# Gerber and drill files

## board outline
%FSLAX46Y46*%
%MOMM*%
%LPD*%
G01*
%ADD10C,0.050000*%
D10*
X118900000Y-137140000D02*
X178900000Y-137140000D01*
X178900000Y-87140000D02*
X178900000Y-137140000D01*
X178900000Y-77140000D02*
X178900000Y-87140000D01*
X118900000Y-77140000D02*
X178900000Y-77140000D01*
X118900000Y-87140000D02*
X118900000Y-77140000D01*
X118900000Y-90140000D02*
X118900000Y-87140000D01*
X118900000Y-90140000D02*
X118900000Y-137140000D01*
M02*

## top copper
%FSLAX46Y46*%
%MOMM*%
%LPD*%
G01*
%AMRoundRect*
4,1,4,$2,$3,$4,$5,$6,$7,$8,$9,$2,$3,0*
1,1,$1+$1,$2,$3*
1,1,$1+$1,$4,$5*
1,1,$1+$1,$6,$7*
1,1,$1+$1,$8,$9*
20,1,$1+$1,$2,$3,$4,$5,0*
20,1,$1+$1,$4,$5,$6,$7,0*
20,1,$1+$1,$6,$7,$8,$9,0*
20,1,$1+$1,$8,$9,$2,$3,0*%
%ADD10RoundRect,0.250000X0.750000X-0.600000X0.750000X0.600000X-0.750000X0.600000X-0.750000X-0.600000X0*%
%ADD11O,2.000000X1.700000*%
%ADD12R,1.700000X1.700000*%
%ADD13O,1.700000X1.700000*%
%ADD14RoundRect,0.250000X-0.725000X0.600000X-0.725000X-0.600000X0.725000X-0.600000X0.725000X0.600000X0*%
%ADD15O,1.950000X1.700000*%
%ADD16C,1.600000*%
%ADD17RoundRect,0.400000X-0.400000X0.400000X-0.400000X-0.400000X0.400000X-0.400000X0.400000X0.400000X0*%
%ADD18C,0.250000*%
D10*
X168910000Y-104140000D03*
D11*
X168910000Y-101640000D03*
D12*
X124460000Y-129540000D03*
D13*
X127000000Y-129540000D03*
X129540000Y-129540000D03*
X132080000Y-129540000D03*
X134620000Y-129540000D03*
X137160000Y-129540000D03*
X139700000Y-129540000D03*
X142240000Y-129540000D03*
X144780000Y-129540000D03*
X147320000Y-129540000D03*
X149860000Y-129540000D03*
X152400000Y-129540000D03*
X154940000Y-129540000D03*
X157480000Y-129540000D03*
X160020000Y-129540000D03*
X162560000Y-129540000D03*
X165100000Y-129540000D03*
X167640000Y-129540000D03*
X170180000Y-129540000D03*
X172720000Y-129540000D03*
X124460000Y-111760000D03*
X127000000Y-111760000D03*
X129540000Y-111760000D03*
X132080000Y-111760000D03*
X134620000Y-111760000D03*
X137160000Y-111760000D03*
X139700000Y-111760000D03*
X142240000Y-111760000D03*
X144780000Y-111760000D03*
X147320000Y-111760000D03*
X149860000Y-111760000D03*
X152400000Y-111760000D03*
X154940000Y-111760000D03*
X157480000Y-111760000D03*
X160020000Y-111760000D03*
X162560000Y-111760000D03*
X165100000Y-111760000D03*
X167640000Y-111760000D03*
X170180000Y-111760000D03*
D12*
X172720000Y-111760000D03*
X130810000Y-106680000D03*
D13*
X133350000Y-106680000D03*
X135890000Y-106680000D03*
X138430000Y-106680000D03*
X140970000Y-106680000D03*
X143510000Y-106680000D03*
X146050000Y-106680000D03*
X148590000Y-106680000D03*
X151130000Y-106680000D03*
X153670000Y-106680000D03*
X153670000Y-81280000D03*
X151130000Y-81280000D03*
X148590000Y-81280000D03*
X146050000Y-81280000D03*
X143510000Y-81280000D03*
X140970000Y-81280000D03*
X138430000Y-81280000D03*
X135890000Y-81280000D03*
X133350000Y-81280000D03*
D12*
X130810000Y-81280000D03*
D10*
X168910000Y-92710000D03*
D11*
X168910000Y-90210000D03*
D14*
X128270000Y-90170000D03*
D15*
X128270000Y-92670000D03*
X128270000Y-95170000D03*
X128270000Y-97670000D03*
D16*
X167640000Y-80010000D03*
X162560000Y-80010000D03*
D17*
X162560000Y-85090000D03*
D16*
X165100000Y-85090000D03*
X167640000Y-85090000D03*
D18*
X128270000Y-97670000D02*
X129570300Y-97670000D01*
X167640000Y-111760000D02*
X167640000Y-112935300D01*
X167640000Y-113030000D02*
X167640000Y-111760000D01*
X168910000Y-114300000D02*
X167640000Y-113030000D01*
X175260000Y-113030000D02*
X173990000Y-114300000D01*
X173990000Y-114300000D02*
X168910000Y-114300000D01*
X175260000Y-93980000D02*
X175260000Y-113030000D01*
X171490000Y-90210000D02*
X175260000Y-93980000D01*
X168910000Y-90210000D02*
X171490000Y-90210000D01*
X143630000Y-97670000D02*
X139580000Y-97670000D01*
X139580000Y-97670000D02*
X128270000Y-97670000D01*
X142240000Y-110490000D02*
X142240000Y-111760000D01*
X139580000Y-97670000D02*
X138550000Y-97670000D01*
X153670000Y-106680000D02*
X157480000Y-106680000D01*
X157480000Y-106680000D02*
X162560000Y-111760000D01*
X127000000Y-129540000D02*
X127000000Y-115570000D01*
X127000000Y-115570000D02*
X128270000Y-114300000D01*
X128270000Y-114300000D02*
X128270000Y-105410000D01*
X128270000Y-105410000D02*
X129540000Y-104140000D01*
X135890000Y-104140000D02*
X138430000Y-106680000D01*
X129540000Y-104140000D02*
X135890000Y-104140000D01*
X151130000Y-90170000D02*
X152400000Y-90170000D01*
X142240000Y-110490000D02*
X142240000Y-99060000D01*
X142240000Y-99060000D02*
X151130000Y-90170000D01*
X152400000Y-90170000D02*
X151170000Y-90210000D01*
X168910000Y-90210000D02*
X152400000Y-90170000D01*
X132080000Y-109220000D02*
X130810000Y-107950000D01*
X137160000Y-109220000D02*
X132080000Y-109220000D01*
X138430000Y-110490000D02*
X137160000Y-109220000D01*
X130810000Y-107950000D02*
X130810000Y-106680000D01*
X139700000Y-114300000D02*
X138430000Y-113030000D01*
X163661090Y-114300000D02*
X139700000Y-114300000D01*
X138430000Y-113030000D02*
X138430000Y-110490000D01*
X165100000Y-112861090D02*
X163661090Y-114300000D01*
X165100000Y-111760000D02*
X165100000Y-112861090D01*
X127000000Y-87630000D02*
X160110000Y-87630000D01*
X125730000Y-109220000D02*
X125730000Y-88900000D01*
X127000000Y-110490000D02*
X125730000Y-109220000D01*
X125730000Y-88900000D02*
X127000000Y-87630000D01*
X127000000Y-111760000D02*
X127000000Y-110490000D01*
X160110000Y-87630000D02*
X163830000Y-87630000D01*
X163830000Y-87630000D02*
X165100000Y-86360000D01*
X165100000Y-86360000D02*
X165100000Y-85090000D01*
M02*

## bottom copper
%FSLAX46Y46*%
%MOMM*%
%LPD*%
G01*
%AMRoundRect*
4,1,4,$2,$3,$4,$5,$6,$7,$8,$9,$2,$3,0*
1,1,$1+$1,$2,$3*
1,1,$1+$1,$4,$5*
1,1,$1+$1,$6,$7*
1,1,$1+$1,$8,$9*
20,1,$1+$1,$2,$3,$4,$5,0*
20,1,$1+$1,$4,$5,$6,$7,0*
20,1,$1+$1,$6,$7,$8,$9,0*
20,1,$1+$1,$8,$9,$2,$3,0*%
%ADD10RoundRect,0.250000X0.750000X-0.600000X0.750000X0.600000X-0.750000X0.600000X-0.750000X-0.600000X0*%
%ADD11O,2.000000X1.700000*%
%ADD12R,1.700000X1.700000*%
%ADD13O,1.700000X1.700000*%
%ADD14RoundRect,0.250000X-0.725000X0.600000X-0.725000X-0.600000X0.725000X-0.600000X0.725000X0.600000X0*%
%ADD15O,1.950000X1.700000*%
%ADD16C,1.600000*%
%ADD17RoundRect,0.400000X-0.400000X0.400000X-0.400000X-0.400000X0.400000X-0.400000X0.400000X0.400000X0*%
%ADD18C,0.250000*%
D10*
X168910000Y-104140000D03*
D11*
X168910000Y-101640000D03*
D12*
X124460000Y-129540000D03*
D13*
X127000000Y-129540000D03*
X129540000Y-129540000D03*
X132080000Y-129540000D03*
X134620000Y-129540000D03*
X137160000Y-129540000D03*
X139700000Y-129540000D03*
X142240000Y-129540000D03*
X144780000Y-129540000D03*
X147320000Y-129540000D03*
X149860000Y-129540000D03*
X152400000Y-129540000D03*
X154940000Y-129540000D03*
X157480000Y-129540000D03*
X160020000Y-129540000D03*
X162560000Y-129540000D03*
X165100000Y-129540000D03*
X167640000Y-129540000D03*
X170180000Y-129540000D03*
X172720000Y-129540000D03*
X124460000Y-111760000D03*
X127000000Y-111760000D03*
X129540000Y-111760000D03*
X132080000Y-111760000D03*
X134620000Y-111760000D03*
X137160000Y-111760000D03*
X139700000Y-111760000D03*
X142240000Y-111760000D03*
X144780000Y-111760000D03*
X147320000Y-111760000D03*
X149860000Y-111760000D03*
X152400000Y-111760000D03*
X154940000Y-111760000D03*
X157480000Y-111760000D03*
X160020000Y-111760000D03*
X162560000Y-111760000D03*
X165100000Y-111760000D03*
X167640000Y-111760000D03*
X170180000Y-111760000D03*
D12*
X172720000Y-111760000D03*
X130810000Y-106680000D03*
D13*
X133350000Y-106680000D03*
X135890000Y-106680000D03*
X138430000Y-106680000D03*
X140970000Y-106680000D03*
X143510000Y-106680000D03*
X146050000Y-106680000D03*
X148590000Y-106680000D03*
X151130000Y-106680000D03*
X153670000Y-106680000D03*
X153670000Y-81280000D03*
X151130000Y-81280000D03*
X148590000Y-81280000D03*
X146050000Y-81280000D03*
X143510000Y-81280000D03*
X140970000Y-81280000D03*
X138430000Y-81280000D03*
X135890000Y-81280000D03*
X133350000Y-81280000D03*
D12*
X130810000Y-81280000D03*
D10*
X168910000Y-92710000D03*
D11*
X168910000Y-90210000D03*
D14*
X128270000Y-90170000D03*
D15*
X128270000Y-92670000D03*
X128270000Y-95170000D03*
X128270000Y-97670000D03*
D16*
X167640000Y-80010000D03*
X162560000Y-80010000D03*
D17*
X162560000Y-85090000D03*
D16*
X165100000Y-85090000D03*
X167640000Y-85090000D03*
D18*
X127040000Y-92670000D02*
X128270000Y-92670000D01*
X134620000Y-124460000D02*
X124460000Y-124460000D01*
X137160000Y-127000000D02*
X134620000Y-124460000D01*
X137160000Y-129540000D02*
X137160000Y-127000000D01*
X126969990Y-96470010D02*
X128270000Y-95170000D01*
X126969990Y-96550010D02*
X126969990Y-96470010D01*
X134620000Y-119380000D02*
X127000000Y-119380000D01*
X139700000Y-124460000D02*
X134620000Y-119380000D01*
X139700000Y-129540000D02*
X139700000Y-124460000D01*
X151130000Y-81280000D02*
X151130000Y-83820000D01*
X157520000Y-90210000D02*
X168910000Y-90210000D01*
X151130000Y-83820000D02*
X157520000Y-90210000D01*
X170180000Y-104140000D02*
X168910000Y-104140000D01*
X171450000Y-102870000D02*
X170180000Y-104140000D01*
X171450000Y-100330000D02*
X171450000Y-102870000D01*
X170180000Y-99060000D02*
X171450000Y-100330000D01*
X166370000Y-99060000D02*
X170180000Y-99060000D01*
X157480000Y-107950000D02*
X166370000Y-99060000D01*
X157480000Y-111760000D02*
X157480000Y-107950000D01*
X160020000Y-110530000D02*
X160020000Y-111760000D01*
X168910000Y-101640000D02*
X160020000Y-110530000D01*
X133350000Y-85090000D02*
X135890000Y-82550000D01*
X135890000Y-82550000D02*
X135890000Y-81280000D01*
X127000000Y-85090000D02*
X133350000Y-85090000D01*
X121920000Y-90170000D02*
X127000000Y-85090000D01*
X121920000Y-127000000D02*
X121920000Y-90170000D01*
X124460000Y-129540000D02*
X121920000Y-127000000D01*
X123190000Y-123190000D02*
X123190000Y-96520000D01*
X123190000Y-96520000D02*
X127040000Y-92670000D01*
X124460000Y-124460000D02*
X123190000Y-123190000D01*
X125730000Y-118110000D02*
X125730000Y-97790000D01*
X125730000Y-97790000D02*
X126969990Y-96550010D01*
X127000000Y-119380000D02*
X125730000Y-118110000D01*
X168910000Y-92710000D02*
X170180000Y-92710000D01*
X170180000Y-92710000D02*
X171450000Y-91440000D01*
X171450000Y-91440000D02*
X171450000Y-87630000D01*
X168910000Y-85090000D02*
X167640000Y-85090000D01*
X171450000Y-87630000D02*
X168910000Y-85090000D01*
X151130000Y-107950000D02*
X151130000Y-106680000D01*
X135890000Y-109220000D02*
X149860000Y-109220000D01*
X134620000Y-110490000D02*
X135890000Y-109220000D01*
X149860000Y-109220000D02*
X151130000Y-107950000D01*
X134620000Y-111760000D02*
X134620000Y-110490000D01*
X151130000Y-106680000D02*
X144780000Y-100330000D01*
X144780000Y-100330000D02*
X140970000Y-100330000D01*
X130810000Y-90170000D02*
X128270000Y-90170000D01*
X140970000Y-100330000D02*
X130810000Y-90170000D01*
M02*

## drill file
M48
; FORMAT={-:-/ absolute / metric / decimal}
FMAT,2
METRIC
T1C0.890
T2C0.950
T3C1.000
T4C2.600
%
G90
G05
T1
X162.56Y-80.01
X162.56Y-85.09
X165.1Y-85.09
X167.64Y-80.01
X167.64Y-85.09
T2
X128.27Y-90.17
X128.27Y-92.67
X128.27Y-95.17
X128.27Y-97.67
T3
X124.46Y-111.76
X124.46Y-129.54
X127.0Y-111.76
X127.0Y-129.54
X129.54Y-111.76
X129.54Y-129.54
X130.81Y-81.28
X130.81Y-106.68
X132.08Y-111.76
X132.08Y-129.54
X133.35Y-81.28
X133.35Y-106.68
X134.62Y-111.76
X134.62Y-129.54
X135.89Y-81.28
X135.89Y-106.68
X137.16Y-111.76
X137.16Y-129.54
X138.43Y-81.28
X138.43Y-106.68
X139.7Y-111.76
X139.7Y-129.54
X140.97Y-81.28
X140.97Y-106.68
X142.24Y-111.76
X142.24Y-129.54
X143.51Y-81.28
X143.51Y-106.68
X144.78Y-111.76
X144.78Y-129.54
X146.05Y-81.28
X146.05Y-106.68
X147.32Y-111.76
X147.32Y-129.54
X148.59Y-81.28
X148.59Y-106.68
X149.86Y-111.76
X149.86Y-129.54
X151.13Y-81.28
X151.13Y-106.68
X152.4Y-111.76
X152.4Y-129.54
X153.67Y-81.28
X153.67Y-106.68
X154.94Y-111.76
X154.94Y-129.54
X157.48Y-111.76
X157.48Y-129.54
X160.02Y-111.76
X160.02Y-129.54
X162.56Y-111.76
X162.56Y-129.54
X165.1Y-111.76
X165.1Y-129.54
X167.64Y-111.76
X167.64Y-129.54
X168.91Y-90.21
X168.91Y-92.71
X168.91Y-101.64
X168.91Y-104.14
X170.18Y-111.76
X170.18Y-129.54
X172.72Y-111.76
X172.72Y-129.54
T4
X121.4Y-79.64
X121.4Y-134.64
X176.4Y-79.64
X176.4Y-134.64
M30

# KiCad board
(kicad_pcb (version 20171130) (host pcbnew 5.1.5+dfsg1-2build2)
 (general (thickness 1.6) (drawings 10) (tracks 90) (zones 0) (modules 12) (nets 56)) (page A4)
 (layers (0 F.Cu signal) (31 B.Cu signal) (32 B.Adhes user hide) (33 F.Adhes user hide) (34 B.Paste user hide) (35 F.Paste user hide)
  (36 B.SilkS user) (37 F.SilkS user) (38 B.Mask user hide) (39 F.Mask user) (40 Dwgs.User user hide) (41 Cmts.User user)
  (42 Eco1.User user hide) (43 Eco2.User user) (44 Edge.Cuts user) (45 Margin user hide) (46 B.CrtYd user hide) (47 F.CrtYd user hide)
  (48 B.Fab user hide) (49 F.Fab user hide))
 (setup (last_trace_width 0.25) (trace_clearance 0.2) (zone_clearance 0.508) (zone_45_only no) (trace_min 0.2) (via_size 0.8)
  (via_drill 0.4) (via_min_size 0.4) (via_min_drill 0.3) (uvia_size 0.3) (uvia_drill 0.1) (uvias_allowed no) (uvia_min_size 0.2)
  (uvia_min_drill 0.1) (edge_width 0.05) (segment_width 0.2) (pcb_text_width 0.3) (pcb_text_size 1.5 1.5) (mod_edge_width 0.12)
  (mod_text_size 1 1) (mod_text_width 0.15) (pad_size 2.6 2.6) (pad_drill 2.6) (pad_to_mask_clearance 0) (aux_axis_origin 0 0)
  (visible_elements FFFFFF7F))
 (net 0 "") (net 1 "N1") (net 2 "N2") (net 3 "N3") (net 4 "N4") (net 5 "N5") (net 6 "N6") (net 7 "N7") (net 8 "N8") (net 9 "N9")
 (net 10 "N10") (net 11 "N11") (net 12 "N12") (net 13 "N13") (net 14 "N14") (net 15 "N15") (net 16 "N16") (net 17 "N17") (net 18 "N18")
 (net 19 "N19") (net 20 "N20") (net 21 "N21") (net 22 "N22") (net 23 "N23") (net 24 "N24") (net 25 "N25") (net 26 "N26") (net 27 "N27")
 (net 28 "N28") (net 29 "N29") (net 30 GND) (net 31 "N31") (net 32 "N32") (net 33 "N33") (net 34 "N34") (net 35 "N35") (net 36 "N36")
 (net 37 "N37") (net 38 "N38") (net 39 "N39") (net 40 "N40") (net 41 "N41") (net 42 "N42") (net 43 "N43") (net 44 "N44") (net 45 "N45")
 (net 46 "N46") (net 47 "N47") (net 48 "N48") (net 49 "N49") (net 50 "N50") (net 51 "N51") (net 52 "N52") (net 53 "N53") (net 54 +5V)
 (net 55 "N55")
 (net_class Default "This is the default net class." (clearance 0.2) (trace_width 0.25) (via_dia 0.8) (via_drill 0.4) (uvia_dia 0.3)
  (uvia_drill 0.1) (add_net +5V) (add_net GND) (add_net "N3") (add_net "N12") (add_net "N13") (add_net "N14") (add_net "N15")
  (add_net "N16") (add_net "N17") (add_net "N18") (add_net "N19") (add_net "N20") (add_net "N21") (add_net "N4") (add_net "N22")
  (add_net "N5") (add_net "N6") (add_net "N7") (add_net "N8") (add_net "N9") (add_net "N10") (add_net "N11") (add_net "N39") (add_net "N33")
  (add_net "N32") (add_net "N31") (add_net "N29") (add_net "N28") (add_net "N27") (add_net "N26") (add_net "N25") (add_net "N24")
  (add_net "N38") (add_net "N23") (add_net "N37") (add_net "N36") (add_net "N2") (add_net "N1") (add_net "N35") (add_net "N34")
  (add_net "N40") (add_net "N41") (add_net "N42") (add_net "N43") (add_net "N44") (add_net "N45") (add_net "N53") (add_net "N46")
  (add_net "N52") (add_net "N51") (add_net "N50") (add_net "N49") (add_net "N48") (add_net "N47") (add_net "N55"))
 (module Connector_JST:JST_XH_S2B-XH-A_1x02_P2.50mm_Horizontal (layer F.Cu) (at 168.91 104.14 90)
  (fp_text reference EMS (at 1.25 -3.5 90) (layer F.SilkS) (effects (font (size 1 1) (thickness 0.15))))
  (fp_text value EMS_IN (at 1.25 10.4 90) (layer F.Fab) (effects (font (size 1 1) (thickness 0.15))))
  (pad 1 thru_hole roundrect (at 0 0 90) (size 1.7 2) (drill 1) (layers *.Cu *.Mask) (roundrect_rratio 0.147059) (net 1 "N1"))
  (pad 2 thru_hole oval (at 2.5 0 90) (size 1.7 2) (drill 1) (layers *.Cu *.Mask) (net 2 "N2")))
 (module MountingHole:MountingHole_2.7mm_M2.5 (layer F.Cu) (at 176.4 134.64)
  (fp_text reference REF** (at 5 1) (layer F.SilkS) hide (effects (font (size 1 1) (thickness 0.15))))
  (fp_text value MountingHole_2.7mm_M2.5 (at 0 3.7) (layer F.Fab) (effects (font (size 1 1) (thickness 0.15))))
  (pad "" np_thru_hole circle (at 0 0) (size 2.6 2.6) (drill 2.6) (layers *.Cu *.Mask)))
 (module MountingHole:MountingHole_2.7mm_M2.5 (layer F.Cu) (at 176.4 79.64)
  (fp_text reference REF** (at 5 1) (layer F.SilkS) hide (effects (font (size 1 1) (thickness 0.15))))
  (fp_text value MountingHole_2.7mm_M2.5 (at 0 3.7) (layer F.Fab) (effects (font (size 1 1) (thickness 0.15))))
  (pad "" np_thru_hole circle (at 0 0) (size 2.6 2.6) (drill 2.6) (layers *.Cu *.Mask)))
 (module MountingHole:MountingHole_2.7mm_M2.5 (layer F.Cu) (at 121.4 79.64)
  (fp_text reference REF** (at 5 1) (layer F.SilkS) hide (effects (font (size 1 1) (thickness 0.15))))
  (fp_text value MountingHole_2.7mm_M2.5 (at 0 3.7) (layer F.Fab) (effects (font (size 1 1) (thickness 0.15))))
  (pad "" np_thru_hole circle (at 0 0) (size 2.6 2.6) (drill 2.6) (layers *.Cu *.Mask)))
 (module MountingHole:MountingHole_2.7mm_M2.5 (layer B.Cu) (at 121.4 134.64)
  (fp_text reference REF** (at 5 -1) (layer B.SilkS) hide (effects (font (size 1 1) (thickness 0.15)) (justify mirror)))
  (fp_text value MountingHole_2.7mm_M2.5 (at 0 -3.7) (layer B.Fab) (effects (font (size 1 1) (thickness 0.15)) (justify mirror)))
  (pad "" np_thru_hole circle (at 0 0) (size 2.6 2.6) (drill 2.6) (layers *.Cu *.Mask)))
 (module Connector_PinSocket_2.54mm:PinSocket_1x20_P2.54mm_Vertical (layer F.Cu) (at 124.46 129.54 90)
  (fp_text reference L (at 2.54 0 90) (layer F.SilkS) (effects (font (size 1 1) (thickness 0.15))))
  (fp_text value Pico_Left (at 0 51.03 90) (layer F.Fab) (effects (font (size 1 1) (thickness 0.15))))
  (pad 1 thru_hole rect (at 0 0 90) (size 1.7 1.7) (drill 1) (layers *.Cu *.Mask) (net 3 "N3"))
  (pad 2 thru_hole oval (at 0 2.54 90) (size 1.7 1.7) (drill 1) (layers *.Cu *.Mask) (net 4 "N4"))
  (pad 3 thru_hole oval (at 0 5.08 90) (size 1.7 1.7) (drill 1) (layers *.Cu *.Mask) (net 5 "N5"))
  (pad 4 thru_hole oval (at 0 7.62 90) (size 1.7 1.7) (drill 1) (layers *.Cu *.Mask) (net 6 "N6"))
  (pad 5 thru_hole oval (at 0 10.16 90) (size 1.7 1.7) (drill 1) (layers *.Cu *.Mask) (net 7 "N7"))
  (pad 6 thru_hole oval (at 0 12.7 90) (size 1.7 1.7) (drill 1) (layers *.Cu *.Mask) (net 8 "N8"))
  (pad 7 thru_hole oval (at 0 15.24 90) (size 1.7 1.7) (drill 1) (layers *.Cu *.Mask) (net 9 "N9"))
  (pad 8 thru_hole oval (at 0 17.78 90) (size 1.7 1.7) (drill 1) (layers *.Cu *.Mask) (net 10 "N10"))
  (pad 9 thru_hole oval (at 0 20.32 90) (size 1.7 1.7) (drill 1) (layers *.Cu *.Mask) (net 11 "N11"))
  (pad 10 thru_hole oval (at 0 22.86 90) (size 1.7 1.7) (drill 1) (layers *.Cu *.Mask) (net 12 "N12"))
  (pad 11 thru_hole oval (at 0 25.4 90) (size 1.7 1.7) (drill 1) (layers *.Cu *.Mask) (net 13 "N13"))
  (pad 12 thru_hole oval (at 0 27.94 90) (size 1.7 1.7) (drill 1) (layers *.Cu *.Mask) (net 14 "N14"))
  (pad 13 thru_hole oval (at 0 30.48 90) (size 1.7 1.7) (drill 1) (layers *.Cu *.Mask) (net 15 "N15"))
  (pad 14 thru_hole oval (at 0 33.02 90) (size 1.7 1.7) (drill 1) (layers *.Cu *.Mask) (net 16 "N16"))
  (pad 15 thru_hole oval (at 0 35.56 90) (size 1.7 1.7) (drill 1) (layers *.Cu *.Mask) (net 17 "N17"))
  (pad 16 thru_hole oval (at 0 38.1 90) (size 1.7 1.7) (drill 1) (layers *.Cu *.Mask) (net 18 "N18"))
  (pad 17 thru_hole oval (at 0 40.64 90) (size 1.7 1.7) (drill 1) (layers *.Cu *.Mask) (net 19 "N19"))
  (pad 18 thru_hole oval (at 0 43.18 90) (size 1.7 1.7) (drill 1) (layers *.Cu *.Mask) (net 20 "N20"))
  (pad 19 thru_hole oval (at 0 45.72 90) (size 1.7 1.7) (drill 1) (layers *.Cu *.Mask) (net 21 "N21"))
  (pad 20 thru_hole oval (at 0 48.26 90) (size 1.7 1.7) (drill 1) (layers *.Cu *.Mask) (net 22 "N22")))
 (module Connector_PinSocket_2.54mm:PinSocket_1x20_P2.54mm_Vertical (layer F.Cu) (at 172.72 111.76 270)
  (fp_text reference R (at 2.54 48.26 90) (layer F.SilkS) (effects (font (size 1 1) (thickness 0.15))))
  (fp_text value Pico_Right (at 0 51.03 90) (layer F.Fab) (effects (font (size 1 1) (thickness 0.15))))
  (pad 20 thru_hole oval (at 0 48.26 270) (size 1.7 1.7) (drill 1) (layers *.Cu *.Mask) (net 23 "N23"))
  (pad 19 thru_hole oval (at 0 45.72 270) (size 1.7 1.7) (drill 1) (layers *.Cu *.Mask) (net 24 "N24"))
  (pad 18 thru_hole oval (at 0 43.18 270) (size 1.7 1.7) (drill 1) (layers *.Cu *.Mask) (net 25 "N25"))
  (pad 17 thru_hole oval (at 0 40.64 270) (size 1.7 1.7) (drill 1) (layers *.Cu *.Mask) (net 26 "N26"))
  (pad 16 thru_hole oval (at 0 38.1 270) (size 1.7 1.7) (drill 1) (layers *.Cu *.Mask) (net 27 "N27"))
  (pad 15 thru_hole oval (at 0 35.56 270) (size 1.7 1.7) (drill 1) (layers *.Cu *.Mask) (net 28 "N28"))
  (pad 14 thru_hole oval (at 0 33.02 270) (size 1.7 1.7) (drill 1) (layers *.Cu *.Mask) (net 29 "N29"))
  (pad 13 thru_hole oval (at 0 30.48 270) (size 1.7 1.7) (drill 1) (layers *.Cu *.Mask) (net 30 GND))
  (pad 12 thru_hole oval (at 0 27.94 270) (size 1.7 1.7) (drill 1) (layers *.Cu *.Mask) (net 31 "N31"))
  (pad 11 thru_hole oval (at 0 25.4 270) (size 1.7 1.7) (drill 1) (layers *.Cu *.Mask) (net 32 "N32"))
  (pad 10 thru_hole oval (at 0 22.86 270) (size 1.7 1.7) (drill 1) (layers *.Cu *.Mask) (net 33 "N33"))
  (pad 9 thru_hole oval (at 0 20.32 270) (size 1.7 1.7) (drill 1) (layers *.Cu *.Mask) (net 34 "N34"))
  (pad 8 thru_hole oval (at 0 17.78 270) (size 1.7 1.7) (drill 1) (layers *.Cu *.Mask) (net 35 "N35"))
  (pad 7 thru_hole oval (at 0 15.24 270) (size 1.7 1.7) (drill 1) (layers *.Cu *.Mask) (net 1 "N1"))
  (pad 6 thru_hole oval (at 0 12.7 270) (size 1.7 1.7) (drill 1) (layers *.Cu *.Mask) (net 2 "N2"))
  (pad 5 thru_hole oval (at 0 10.16 270) (size 1.7 1.7) (drill 1) (layers *.Cu *.Mask) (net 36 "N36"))
  (pad 4 thru_hole oval (at 0 7.62 270) (size 1.7 1.7) (drill 1) (layers *.Cu *.Mask) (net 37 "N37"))
  (pad 3 thru_hole oval (at 0 5.08 270) (size 1.7 1.7) (drill 1) (layers *.Cu *.Mask) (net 30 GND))
  (pad 2 thru_hole oval (at 0 2.54 270) (size 1.7 1.7) (drill 1) (layers *.Cu *.Mask) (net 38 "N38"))
  (pad 1 thru_hole rect (at 0 0 270) (size 1.7 1.7) (drill 1) (layers *.Cu *.Mask) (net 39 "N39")))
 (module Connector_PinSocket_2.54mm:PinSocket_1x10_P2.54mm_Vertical (layer F.Cu) (at 130.81 106.68 90)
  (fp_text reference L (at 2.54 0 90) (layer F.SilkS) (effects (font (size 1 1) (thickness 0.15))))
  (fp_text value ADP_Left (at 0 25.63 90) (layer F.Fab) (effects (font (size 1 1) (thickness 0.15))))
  (pad 1 thru_hole rect (at 0 0 90) (size 1.7 1.7) (drill 1) (layers *.Cu *.Mask) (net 37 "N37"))
  (pad 2 thru_hole oval (at 0 2.54 90) (size 1.7 1.7) (drill 1) (layers *.Cu *.Mask) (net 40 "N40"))
  (pad 3 thru_hole oval (at 0 5.08 90) (size 1.7 1.7) (drill 1) (layers *.Cu *.Mask) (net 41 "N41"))
  (pad 4 thru_hole oval (at 0 7.62 90) (size 1.7 1.7) (drill 1) (layers *.Cu *.Mask) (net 4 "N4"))
  (pad 5 thru_hole oval (at 0 10.16 90) (size 1.7 1.7) (drill 1) (layers *.Cu *.Mask) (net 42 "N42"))
  (pad 6 thru_hole oval (at 0 12.7 90) (size 1.7 1.7) (drill 1) (layers *.Cu *.Mask) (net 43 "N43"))
  (pad 7 thru_hole oval (at 0 15.24 90) (size 1.7 1.7) (drill 1) (layers *.Cu *.Mask) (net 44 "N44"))
  (pad 8 thru_hole oval (at 0 17.78 90) (size 1.7 1.7) (drill 1) (layers *.Cu *.Mask) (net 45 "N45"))
  (pad 9 thru_hole oval (at 0 20.32 90) (size 1.7 1.7) (drill 1) (layers *.Cu *.Mask) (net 27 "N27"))
  (pad 10 thru_hole oval (at 0 22.86 90) (size 1.7 1.7) (drill 1) (layers *.Cu *.Mask) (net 36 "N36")))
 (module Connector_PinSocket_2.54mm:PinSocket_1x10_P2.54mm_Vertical (layer F.Cu) (at 130.81 81.28 90)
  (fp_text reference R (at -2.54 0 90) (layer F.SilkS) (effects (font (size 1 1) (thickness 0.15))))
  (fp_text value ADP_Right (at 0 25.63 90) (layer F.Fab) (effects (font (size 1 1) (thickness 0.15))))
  (pad 10 thru_hole oval (at 0 22.86 90) (size 1.7 1.7) (drill 1) (layers *.Cu *.Mask) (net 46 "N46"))
  (pad 9 thru_hole oval (at 0 20.32 90) (size 1.7 1.7) (drill 1) (layers *.Cu *.Mask) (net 30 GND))
  (pad 8 thru_hole oval (at 0 17.78 90) (size 1.7 1.7) (drill 1) (layers *.Cu *.Mask) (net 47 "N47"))
  (pad 7 thru_hole oval (at 0 15.24 90) (size 1.7 1.7) (drill 1) (layers *.Cu *.Mask) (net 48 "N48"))
  (pad 6 thru_hole oval (at 0 12.7 90) (size 1.7 1.7) (drill 1) (layers *.Cu *.Mask) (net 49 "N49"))
  (pad 5 thru_hole oval (at 0 10.16 90) (size 1.7 1.7) (drill 1) (layers *.Cu *.Mask) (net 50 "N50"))
  (pad 4 thru_hole oval (at 0 7.62 90) (size 1.7 1.7) (drill 1) (layers *.Cu *.Mask) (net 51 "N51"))
  (pad 3 thru_hole oval (at 0 5.08 90) (size 1.7 1.7) (drill 1) (layers *.Cu *.Mask) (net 3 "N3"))
  (pad 2 thru_hole oval (at 0 2.54 90) (size 1.7 1.7) (drill 1) (layers *.Cu *.Mask) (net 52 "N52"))
  (pad 1 thru_hole rect (at 0 0 90) (size 1.7 1.7) (drill 1) (layers *.Cu *.Mask) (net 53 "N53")))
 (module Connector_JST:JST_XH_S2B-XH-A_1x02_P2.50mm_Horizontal (layer F.Cu) (at 168.91 92.71 90)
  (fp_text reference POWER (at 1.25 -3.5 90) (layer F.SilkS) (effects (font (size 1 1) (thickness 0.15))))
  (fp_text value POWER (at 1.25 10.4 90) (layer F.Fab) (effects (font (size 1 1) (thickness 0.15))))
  (pad 1 thru_hole roundrect (at 0 0 90) (size 1.7 2) (drill 1) (layers *.Cu *.Mask) (roundrect_rratio 0.1470588235294118) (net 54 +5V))
  (pad 2 thru_hole oval (at 2.5 0 90) (size 1.7 2) (drill 1) (layers *.Cu *.Mask) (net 30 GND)))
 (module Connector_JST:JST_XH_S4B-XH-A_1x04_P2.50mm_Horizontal (layer F.Cu) (at 128.27 90.17 270)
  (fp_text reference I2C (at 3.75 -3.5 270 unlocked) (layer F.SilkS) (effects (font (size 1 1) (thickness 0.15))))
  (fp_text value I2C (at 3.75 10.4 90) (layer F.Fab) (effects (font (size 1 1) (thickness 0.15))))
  (pad 1 thru_hole roundrect (at 0 0 270) (size 1.7 1.95) (drill 0.95) (layers *.Cu *.Mask) (roundrect_rratio 0.147059) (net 27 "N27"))
  (pad 2 thru_hole oval (at 2.5 0 270) (size 1.7 1.95) (drill 0.95) (layers *.Cu *.Mask) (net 8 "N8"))
  (pad 3 thru_hole oval (at 5 0 270) (size 1.7 1.95) (drill 0.95) (layers *.Cu *.Mask) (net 9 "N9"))
  (pad 4 thru_hole oval (at 7.5 0 270) (size 1.7 1.95) (drill 0.95) (layers *.Cu *.Mask) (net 30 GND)))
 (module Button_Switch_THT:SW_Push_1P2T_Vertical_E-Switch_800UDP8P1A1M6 (layer F.Cu) (at 162.56 85.09 90)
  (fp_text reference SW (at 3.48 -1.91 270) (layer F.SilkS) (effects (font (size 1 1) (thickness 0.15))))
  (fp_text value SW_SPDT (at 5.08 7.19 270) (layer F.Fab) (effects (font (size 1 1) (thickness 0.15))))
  (pad "" thru_hole circle (at 5.08 5.08 270) (size 1.6 1.6) (drill 0.89) (layers *.Cu *.Mask))
  (pad "" thru_hole circle (at 5.08 0 270) (size 1.6 1.6) (drill 0.89) (layers *.Cu *.Mask))
  (pad 1 thru_hole roundrect (at 0 0 270) (size 1.6 1.6) (drill 0.89) (layers *.Cu *.Mask) (roundrect_rratio 0.25) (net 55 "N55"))
  (pad 2 thru_hole circle (at 0 2.54 270) (size 1.6 1.6) (drill 0.89) (layers *.Cu *.Mask) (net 24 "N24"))
  (pad 3 thru_hole circle (at 0 5.08 270) (size 1.6 1.6) (drill 0.89) (layers *.Cu *.Mask) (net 54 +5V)))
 (gr_line (start 118.9 137.14) (end 178.9 137.14) (layer Edge.Cuts) (width 0.05))
 (gr_line (start 178.9 87.14) (end 178.9 137.14) (layer Edge.Cuts) (width 0.05))
 (gr_line (start 178.9 77.14) (end 178.9 87.14) (layer Edge.Cuts) (width 0.05))
 (gr_line (start 118.9 77.14) (end 178.9 77.14) (layer Edge.Cuts) (width 0.05))
 (gr_line (start 118.9 87.14) (end 118.9 77.14) (layer Edge.Cuts) (width 0.05))
 (gr_line (start 118.9 90.14) (end 118.9 87.14) (layer Edge.Cuts) (width 0.05))
 (gr_line (start 118.9 90.14) (end 118.9 137.14) (layer Edge.Cuts) (width 0.05))
 (segment (start 127.04 92.67) (end 128.27 92.67) (width 0.25) (layer B.Cu) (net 8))
 (segment (start 134.62 124.46) (end 124.46 124.46) (width 0.25) (layer B.Cu) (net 8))
 (segment (start 137.16 127) (end 134.62 124.46) (width 0.25) (layer B.Cu) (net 8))
 (segment (start 137.16 129.54) (end 137.16 127) (width 0.25) (layer B.Cu) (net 8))
 (segment (start 126.96999 96.47001) (end 128.27 95.17) (width 0.25) (layer B.Cu) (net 9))
 (segment (start 126.96999 96.55001) (end 126.96999 96.47001) (width 0.25) (layer B.Cu) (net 9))
 (segment (start 134.62 119.38) (end 127 119.38) (width 0.25) (layer B.Cu) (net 9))
 (segment (start 139.7 124.46) (end 134.62 119.38) (width 0.25) (layer B.Cu) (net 9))
 (segment (start 139.7 129.54) (end 139.7 124.46) (width 0.25) (layer B.Cu) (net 9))
 (segment (start 128.27 97.67) (end 129.5703 97.67) (width 0.25) (layer F.Cu) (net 30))
 (segment (start 167.64 111.76) (end 167.64 112.9353) (width 0.25) (layer F.Cu) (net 30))
 (segment (start 151.13 81.28) (end 151.13 83.82) (width 0.25) (layer B.Cu) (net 30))
 (segment (start 157.52 90.21) (end 168.91 90.21) (width 0.25) (layer B.Cu) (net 30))
 (segment (start 151.13 83.82) (end 157.52 90.21) (width 0.25) (layer B.Cu) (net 30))
 (segment (start 167.64 113.03) (end 167.64 111.76) (width 0.25) (layer F.Cu) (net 30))
 (segment (start 168.91 114.3) (end 167.64 113.03) (width 0.25) (layer F.Cu) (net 30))
 (segment (start 175.26 113.03) (end 173.99 114.3) (width 0.25) (layer F.Cu) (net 30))
 (segment (start 173.99 114.3) (end 168.91 114.3) (width 0.25) (layer F.Cu) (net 30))
 (segment (start 175.26 93.98) (end 175.26 113.03) (width 0.25) (layer F.Cu) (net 30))
 (segment (start 171.49 90.21) (end 175.26 93.98) (width 0.25) (layer F.Cu) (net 30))
 (segment (start 168.91 90.21) (end 171.49 90.21) (width 0.25) (layer F.Cu) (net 30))
 (segment (start 143.63 97.67) (end 139.58 97.67) (width 0.25) (layer F.Cu) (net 30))
 (segment (start 139.58 97.67) (end 128.27 97.67) (width 0.25) (layer F.Cu) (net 30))
 (segment (start 142.24 110.49) (end 142.24 111.76) (width 0.25) (layer F.Cu) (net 30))
 (segment (start 139.58 97.67) (end 138.55 97.67) (width 0.25) (layer F.Cu) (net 30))
 (segment (start 170.18 104.14) (end 168.91 104.14) (width 0.25) (layer B.Cu) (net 1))
 (segment (start 171.45 102.87) (end 170.18 104.14) (width 0.25) (layer B.Cu) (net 1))
 (segment (start 171.45 100.33) (end 171.45 102.87) (width 0.25) (layer B.Cu) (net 1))
 (segment (start 170.18 99.06) (end 171.45 100.33) (width 0.25) (layer B.Cu) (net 1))
 (segment (start 166.37 99.06) (end 170.18 99.06) (width 0.25) (layer B.Cu) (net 1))
 (segment (start 157.48 107.95) (end 166.37 99.06) (width 0.25) (layer B.Cu) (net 1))
 (segment (start 157.48 111.76) (end 157.48 107.95) (width 0.25) (layer B.Cu) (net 1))
 (segment (start 160.02 110.53) (end 160.02 111.76) (width 0.25) (layer B.Cu) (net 2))
 (segment (start 168.91 101.64) (end 160.02 110.53) (width 0.25) (layer B.Cu) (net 2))
 (segment (start 153.67 106.68) (end 157.48 106.68) (width 0.25) (layer F.Cu) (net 36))
 (segment (start 157.48 106.68) (end 162.56 111.76) (width 0.25) (layer F.Cu) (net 36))
 (segment (start 133.35 85.09) (end 135.89 82.55) (width 0.25) (layer B.Cu) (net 3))
 (segment (start 135.89 82.55) (end 135.89 81.28) (width 0.25) (layer B.Cu) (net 3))
 (segment (start 127 85.09) (end 133.35 85.09) (width 0.25) (layer B.Cu) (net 3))
 (segment (start 121.92 90.17) (end 127 85.09) (width 0.25) (layer B.Cu) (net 3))
 (segment (start 121.92 127) (end 121.92 90.17) (width 0.25) (layer B.Cu) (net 3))
 (segment (start 124.46 129.54) (end 121.92 127) (width 0.25) (layer B.Cu) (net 3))
 (segment (start 127 129.54) (end 127 115.57) (width 0.25) (layer F.Cu) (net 4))
 (segment (start 127 115.57) (end 128.27 114.3) (width 0.25) (layer F.Cu) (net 4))
 (segment (start 128.27 114.3) (end 128.27 105.41) (width 0.25) (layer F.Cu) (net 4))
 (segment (start 128.27 105.41) (end 129.54 104.14) (width 0.25) (layer F.Cu) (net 4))
 (segment (start 135.89 104.14) (end 138.43 106.68) (width 0.25) (layer F.Cu) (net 4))
 (segment (start 129.54 104.14) (end 135.89 104.14) (width 0.25) (layer F.Cu) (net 4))
 (segment (start 123.19 123.19) (end 123.19 96.52) (width 0.25) (layer B.Cu) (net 8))
 (segment (start 123.19 96.52) (end 127.04 92.67) (width 0.25) (layer B.Cu) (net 8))
 (segment (start 124.46 124.46) (end 123.19 123.19) (width 0.25) (layer B.Cu) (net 8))
 (segment (start 125.73 118.11) (end 125.73 97.79) (width 0.25) (layer B.Cu) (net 9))
 (segment (start 125.73 97.79) (end 126.96999 96.55001) (width 0.25) (layer B.Cu) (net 9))
 (segment (start 127 119.38) (end 125.73 118.11) (width 0.25) (layer B.Cu) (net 9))
 (segment (start 151.13 90.17) (end 152.4 90.17) (width 0.25) (layer F.Cu) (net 30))
 (segment (start 142.24 110.49) (end 142.24 99.06) (width 0.25) (layer F.Cu) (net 30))
 (segment (start 142.24 99.06) (end 151.13 90.17) (width 0.25) (layer F.Cu) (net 30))
 (segment (start 152.4 90.17) (end 151.17 90.21) (width 0.25) (layer F.Cu) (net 30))
 (segment (start 168.91 90.21) (end 152.4 90.17) (width 0.25) (layer F.Cu) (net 30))
 (segment (start 132.08 109.22) (end 130.81 107.95) (width 0.25) (layer F.Cu) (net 37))
 (segment (start 137.16 109.22) (end 132.08 109.22) (width 0.25) (layer F.Cu) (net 37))
 (segment (start 138.43 110.49) (end 137.16 109.22) (width 0.25) (layer F.Cu) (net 37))
 (segment (start 130.81 107.95) (end 130.81 106.68) (width 0.25) (layer F.Cu) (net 37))
 (segment (start 139.7 114.3) (end 138.43 113.03) (width 0.25) (layer F.Cu) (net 37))
 (segment (start 163.66109 114.3) (end 139.7 114.3) (width 0.25) (layer F.Cu) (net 37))
 (segment (start 138.43 113.03) (end 138.43 110.49) (width 0.25) (layer F.Cu) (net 37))
 (segment (start 165.1 112.86109) (end 163.66109 114.3) (width 0.25) (layer F.Cu) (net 37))
 (segment (start 165.1 111.76) (end 165.1 112.86109) (width 0.25) (layer F.Cu) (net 37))
 (segment (start 168.91 92.71) (end 170.18 92.71) (width 0.25) (layer B.Cu) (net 54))
 (segment (start 170.18 92.71) (end 171.45 91.44) (width 0.25) (layer B.Cu) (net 54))
 (segment (start 171.45 91.44) (end 171.45 87.63) (width 0.25) (layer B.Cu) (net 54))
 (segment (start 168.91 85.09) (end 167.64 85.09) (width 0.25) (layer B.Cu) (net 54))
 (segment (start 171.45 87.63) (end 168.91 85.09) (width 0.25) (layer B.Cu) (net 54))
 (segment (start 151.13 107.95) (end 151.13 106.68) (width 0.25) (layer B.Cu) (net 27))
 (segment (start 135.89 109.22) (end 149.86 109.22) (width 0.25) (layer B.Cu) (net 27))
 (segment (start 134.62 110.49) (end 135.89 109.22) (width 0.25) (layer B.Cu) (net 27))
 (segment (start 149.86 109.22) (end 151.13 107.95) (width 0.25) (layer B.Cu) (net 27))
 (segment (start 134.62 111.76) (end 134.62 110.49) (width 0.25) (layer B.Cu) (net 27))
 (segment (start 151.13 106.68) (end 144.78 100.33) (width 0.25) (layer B.Cu) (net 27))
 (segment (start 144.78 100.33) (end 140.97 100.33) (width 0.25) (layer B.Cu) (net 27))
 (segment (start 130.81 90.17) (end 128.27 90.17) (width 0.25) (layer B.Cu) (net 27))
 (segment (start 140.97 100.33) (end 130.81 90.17) (width 0.25) (layer B.Cu) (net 27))
 (segment (start 127 87.63) (end 160.11 87.63) (width 0.25) (layer F.Cu) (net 24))
 (segment (start 125.73 109.22) (end 125.73 88.9) (width 0.25) (layer F.Cu) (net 24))
 (segment (start 127 110.49) (end 125.73 109.22) (width 0.25) (layer F.Cu) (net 24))
 (segment (start 125.73 88.9) (end 127 87.63) (width 0.25) (layer F.Cu) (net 24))
 (segment (start 127 111.76) (end 127 110.49) (width 0.25) (layer F.Cu) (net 24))
 (segment (start 160.11 87.63) (end 163.83 87.63) (width 0.25) (layer F.Cu) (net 24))
 (segment (start 163.83 87.63) (end 165.1 86.36) (width 0.25) (layer F.Cu) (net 24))
 (segment (start 165.1 86.36) (end 165.1 85.09) (width 0.25) (layer F.Cu) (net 24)))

